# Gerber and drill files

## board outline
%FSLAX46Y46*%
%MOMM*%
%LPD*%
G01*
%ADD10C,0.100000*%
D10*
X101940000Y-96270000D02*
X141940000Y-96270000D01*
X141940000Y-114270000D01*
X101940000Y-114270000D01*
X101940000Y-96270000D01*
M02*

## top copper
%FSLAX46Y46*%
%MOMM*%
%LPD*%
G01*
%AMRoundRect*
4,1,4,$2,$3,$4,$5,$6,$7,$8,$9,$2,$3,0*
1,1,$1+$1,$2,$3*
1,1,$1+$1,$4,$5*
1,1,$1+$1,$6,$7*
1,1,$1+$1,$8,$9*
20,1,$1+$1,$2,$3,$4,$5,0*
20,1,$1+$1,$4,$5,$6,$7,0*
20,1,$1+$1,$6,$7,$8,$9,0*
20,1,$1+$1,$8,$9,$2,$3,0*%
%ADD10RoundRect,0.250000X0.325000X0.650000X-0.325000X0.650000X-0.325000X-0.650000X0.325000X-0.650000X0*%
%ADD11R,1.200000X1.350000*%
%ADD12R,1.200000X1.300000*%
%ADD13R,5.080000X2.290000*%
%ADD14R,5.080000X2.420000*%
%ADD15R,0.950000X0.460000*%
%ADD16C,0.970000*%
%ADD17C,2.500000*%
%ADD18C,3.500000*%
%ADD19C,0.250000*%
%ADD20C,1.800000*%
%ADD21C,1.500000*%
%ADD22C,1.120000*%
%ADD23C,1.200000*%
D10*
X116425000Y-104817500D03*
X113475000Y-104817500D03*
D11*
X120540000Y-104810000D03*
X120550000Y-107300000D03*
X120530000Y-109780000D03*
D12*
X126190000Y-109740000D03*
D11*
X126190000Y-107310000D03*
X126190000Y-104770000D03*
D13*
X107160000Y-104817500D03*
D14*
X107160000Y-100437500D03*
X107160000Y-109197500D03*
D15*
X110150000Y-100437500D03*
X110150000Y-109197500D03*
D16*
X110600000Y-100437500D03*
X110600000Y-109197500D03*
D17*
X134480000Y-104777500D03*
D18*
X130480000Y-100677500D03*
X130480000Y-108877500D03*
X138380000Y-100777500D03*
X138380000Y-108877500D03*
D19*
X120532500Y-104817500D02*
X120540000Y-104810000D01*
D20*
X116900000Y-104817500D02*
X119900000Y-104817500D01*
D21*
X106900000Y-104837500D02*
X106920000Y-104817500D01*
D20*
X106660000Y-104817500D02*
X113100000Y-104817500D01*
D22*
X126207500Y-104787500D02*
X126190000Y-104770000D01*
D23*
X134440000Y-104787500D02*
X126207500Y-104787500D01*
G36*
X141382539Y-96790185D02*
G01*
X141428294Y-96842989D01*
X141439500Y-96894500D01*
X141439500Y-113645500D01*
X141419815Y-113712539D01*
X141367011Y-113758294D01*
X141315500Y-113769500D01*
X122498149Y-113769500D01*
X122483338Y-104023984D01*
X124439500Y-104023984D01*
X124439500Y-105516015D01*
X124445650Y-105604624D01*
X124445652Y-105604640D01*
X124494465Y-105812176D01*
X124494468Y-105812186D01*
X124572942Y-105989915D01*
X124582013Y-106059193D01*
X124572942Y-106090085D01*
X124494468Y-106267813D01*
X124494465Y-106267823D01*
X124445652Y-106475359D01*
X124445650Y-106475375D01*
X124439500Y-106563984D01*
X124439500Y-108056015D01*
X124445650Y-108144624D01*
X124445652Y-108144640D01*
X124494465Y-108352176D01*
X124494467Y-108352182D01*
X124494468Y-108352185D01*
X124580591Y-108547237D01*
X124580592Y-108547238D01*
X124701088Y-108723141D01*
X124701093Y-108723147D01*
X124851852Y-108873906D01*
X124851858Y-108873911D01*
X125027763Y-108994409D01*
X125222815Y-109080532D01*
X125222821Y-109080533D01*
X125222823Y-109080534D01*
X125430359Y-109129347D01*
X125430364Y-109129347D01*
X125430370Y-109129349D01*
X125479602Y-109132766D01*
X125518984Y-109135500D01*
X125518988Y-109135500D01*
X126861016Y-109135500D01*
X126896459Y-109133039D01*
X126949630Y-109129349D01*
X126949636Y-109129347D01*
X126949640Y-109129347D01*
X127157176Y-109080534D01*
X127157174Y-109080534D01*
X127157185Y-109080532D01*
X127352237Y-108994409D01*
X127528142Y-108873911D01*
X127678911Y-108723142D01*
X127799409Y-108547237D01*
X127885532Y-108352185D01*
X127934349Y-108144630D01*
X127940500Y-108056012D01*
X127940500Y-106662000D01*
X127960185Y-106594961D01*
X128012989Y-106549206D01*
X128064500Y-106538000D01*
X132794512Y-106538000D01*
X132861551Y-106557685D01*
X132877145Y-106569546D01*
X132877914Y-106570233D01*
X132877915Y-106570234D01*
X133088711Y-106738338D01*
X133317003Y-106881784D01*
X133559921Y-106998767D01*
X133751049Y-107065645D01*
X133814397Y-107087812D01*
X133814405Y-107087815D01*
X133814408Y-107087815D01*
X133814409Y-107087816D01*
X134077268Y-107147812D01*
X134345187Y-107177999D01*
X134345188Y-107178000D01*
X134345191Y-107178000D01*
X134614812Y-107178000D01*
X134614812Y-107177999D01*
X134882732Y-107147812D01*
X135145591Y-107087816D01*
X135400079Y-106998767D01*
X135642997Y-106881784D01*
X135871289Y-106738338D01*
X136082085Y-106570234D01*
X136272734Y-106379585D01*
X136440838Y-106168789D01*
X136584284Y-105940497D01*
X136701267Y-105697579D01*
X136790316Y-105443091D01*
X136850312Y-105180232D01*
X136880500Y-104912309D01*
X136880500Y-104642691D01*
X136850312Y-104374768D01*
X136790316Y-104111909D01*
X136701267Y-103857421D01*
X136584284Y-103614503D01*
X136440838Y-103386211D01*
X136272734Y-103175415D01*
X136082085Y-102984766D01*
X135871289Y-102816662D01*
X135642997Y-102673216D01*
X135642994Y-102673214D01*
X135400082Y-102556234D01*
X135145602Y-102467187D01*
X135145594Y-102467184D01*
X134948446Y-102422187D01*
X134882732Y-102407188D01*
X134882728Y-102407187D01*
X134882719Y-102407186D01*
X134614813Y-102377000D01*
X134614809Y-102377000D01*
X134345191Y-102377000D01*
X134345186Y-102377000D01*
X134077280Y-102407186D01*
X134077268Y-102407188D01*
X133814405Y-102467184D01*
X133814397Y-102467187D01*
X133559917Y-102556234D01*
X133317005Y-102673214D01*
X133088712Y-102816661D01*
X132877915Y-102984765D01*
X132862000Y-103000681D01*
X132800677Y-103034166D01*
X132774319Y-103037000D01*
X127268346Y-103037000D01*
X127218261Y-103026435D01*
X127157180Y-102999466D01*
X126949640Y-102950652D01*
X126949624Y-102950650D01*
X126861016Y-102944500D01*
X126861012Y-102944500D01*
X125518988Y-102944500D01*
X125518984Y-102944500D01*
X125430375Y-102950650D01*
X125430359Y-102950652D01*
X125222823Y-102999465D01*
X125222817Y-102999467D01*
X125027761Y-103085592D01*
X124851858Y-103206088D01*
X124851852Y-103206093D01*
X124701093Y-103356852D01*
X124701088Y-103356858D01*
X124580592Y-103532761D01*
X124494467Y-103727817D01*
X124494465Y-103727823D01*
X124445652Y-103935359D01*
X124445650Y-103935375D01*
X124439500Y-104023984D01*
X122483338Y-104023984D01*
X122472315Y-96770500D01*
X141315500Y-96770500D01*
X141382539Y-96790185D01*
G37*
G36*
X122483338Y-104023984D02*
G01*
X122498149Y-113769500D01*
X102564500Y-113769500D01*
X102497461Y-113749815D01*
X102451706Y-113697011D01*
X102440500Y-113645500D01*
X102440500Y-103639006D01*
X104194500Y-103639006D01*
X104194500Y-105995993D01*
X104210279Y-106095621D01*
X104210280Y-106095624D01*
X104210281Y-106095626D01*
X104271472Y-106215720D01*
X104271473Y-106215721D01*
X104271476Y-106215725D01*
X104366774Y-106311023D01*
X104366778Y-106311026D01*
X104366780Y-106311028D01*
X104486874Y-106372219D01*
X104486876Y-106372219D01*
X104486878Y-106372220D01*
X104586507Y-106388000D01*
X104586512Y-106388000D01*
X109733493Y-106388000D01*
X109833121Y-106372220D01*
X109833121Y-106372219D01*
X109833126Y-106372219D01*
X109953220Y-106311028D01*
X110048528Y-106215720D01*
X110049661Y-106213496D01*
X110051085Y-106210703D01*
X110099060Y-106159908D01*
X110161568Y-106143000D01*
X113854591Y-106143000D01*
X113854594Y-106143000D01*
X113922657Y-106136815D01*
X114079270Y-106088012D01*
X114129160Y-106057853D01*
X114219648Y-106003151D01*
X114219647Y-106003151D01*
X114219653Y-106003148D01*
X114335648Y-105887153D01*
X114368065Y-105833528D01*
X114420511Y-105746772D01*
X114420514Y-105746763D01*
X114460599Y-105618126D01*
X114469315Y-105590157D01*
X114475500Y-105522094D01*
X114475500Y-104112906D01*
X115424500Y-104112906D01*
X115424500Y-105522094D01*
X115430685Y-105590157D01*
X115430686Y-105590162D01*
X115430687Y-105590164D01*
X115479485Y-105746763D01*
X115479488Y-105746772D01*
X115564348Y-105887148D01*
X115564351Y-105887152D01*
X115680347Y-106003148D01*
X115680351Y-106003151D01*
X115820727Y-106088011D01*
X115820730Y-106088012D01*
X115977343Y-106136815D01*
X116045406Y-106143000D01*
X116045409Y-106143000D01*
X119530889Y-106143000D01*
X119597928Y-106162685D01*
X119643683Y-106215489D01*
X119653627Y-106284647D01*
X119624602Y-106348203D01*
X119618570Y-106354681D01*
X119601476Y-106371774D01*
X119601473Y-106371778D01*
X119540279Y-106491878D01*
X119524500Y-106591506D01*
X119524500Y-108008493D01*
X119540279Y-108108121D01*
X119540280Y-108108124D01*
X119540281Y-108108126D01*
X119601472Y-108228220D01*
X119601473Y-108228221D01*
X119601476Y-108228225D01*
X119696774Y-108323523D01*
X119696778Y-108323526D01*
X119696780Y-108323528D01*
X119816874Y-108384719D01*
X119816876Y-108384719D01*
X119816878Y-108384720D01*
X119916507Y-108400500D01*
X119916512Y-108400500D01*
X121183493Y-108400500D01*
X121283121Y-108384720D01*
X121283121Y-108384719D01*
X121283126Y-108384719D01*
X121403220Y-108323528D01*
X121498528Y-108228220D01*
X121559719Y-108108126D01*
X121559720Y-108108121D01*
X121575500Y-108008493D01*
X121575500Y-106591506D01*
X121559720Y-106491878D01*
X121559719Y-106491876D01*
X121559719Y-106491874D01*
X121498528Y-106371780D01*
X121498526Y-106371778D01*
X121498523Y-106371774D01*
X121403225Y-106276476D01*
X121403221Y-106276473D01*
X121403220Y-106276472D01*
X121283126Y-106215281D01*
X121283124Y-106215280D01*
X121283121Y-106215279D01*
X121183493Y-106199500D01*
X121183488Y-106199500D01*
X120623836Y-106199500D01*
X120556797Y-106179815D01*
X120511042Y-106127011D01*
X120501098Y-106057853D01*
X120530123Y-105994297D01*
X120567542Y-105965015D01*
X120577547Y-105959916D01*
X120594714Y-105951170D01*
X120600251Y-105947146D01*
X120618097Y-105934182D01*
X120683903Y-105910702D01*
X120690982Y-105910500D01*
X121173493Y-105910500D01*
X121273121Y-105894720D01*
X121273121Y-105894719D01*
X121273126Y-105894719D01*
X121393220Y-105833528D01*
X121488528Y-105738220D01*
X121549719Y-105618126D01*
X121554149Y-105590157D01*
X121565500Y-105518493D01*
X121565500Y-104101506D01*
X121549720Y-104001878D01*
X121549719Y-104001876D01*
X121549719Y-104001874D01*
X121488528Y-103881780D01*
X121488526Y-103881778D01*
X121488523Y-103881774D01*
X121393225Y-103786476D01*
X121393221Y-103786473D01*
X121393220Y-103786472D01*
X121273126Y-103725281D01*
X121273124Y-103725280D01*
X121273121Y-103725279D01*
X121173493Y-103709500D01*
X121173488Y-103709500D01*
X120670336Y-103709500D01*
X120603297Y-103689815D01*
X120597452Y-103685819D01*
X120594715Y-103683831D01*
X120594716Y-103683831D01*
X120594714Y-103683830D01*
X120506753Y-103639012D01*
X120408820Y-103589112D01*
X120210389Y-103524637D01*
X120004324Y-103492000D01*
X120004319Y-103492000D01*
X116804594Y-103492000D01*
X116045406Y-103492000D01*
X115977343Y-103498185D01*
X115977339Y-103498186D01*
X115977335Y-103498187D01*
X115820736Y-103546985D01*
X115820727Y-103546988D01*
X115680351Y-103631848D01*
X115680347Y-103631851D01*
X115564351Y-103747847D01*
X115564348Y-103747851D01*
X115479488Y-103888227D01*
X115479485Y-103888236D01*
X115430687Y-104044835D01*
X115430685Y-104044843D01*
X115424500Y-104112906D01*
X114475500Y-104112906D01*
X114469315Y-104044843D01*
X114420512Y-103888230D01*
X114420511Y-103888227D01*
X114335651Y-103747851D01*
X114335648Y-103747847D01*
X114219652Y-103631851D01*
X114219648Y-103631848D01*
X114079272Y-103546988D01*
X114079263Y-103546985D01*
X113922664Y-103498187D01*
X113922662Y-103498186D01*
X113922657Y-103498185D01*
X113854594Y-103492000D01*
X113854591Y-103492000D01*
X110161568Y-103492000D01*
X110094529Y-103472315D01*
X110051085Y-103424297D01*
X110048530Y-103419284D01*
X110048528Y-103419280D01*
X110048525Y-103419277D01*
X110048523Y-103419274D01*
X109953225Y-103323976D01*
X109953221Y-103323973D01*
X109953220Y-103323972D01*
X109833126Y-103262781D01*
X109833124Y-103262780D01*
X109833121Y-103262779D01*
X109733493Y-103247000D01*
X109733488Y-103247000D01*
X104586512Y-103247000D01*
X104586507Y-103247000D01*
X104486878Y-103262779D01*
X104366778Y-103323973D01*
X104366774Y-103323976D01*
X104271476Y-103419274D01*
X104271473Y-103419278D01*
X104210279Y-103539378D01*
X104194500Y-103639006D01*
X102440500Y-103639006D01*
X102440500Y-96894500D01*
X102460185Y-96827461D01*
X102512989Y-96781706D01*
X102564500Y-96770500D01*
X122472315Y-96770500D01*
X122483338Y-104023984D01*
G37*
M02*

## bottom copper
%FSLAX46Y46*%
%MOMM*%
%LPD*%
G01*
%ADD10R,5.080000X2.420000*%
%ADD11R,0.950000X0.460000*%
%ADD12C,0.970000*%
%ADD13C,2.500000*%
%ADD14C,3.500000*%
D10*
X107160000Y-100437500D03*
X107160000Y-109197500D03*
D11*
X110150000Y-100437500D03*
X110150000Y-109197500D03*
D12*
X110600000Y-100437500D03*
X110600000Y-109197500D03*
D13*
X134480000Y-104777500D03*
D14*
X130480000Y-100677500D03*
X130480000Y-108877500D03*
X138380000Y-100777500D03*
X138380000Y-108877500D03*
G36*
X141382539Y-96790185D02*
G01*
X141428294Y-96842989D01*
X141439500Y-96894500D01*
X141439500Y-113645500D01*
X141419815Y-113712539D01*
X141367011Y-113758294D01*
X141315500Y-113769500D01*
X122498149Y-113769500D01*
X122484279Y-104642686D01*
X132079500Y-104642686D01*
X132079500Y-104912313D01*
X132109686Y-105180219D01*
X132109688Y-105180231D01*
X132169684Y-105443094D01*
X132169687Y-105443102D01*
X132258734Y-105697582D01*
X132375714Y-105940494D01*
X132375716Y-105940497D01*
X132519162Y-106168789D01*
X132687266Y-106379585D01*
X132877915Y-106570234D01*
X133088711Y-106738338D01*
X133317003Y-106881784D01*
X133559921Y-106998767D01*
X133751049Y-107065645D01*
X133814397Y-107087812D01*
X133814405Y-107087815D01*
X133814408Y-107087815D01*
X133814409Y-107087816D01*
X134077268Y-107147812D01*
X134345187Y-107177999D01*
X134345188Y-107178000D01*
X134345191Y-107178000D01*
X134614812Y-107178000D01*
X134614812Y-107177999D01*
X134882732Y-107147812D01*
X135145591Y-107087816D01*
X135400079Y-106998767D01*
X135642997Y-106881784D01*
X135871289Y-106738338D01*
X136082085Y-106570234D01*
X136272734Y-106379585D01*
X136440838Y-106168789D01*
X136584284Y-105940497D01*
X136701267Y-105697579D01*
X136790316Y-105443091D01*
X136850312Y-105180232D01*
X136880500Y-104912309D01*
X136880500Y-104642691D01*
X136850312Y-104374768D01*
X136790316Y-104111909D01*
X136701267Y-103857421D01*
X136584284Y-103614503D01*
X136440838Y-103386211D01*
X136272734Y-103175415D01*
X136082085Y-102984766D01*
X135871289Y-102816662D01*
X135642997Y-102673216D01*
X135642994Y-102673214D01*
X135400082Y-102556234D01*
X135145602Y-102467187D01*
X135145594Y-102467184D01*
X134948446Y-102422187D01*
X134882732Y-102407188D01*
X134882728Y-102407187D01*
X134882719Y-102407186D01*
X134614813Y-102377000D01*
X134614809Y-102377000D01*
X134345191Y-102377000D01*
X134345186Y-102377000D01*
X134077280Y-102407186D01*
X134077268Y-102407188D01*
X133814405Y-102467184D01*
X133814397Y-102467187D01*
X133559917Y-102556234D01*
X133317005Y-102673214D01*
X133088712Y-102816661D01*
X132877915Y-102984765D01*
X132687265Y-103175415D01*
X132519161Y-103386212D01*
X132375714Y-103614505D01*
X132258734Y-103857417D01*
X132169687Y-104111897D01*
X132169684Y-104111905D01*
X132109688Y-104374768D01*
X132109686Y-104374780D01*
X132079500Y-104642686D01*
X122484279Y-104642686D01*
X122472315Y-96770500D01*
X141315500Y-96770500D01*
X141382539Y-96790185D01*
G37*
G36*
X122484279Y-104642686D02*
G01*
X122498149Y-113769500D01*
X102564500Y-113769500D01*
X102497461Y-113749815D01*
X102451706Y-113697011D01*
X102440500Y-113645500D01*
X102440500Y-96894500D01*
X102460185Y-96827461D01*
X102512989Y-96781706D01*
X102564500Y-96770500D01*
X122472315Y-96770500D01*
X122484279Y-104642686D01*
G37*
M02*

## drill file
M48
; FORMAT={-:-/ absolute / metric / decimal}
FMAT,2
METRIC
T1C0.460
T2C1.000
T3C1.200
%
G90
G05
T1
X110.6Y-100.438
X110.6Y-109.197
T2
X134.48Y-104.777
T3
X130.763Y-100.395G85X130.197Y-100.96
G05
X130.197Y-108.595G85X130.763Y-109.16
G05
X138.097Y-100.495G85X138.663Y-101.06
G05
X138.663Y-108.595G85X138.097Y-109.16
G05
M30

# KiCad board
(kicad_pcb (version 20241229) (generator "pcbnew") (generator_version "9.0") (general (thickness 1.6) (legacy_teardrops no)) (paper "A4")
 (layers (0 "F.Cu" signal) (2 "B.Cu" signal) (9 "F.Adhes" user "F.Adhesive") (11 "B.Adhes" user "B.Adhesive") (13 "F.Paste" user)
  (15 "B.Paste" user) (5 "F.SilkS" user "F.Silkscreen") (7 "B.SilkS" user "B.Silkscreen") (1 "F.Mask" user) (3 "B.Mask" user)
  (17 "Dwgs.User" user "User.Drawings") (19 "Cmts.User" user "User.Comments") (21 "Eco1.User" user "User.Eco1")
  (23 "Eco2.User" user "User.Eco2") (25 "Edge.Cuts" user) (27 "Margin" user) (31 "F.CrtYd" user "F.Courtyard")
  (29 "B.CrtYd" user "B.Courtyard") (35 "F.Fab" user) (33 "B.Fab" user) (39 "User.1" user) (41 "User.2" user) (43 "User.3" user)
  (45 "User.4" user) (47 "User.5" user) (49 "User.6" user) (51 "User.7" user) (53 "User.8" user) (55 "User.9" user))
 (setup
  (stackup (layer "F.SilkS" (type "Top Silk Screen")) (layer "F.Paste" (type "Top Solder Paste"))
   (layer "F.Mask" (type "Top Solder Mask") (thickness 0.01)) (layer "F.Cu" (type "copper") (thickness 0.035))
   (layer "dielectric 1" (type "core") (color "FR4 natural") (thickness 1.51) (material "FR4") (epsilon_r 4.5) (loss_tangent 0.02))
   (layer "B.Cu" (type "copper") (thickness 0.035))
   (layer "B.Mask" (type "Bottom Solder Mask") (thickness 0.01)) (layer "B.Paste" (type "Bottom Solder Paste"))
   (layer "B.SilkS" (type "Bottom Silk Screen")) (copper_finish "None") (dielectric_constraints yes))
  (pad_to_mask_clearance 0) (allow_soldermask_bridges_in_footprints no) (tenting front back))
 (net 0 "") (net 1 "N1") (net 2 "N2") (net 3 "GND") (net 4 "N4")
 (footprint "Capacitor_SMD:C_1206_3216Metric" (layer "F.Cu") (at 114.95 104.8175 180)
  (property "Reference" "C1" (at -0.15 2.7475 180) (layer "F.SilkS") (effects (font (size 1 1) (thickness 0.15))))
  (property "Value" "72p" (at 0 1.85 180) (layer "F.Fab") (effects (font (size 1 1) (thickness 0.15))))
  (pad "1" smd roundrect (at -1.475 0 180) (size 1.15 1.8) (layers "F.Cu" "F.Mask" "F.Paste") (roundrect_rratio 0.217391) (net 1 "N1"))
  (pad "2" smd roundrect (at 1.475 0 180) (size 1.15 1.8) (layers "F.Cu" "F.Mask" "F.Paste") (roundrect_rratio 0.217391) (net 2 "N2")))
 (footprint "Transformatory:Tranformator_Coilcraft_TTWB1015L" (layer "F.Cu") (at 120.16 104.23)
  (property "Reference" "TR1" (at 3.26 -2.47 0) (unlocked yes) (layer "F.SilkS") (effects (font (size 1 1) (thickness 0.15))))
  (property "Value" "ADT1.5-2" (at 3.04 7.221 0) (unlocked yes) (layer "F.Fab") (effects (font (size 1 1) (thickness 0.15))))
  (pad "1" smd rect (at 0.38 0.58) (size 1.2 1.35) (layers "F.Cu" "F.Mask" "F.Paste") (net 1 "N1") (thermal_bridge_angle 45))
  (pad "2" smd rect (at 0.39 3.07) (size 1.2 1.35) (layers "F.Cu" "F.Mask" "F.Paste") (thermal_bridge_angle 45))
  (pad "3" smd rect (at 0.37 5.55) (size 1.2 1.35) (layers "F.Cu" "F.Mask" "F.Paste") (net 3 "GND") (thermal_bridge_angle 45))
  (pad "4" smd rect (at 6.03 5.51) (size 1.2 1.3) (layers "F.Cu" "F.Mask" "F.Paste") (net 3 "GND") (thermal_bridge_angle 45))
  (pad "5" smd rect (at 6.03 3.08) (size 1.2 1.35) (layers "F.Cu" "F.Mask" "F.Paste") (thermal_bridge_angle 45))
  (pad "6" smd rect (at 6.03 0.54) (size 1.2 1.35) (layers "F.Cu" "F.Mask" "F.Paste") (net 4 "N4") (thermal_bridge_angle 45)))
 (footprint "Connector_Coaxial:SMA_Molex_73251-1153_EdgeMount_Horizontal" (layer "F.Cu") (at 108.88 104.8175)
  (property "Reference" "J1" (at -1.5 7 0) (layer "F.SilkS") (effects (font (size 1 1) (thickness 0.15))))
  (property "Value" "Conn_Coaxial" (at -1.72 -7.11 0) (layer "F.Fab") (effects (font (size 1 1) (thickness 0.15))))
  (pad "1" smd rect (at -1.72 0) (size 5.08 2.29) (layers "F.Cu" "F.Mask" "F.Paste") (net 2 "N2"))
  (pad "2" smd rect (at -1.72 -4.38) (size 5.08 2.42) (layers "F.Cu" "F.Mask" "F.Paste") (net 3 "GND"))
  (pad "2" smd rect (at -1.72 -4.38) (size 5.08 2.42) (layers "B.Cu" "B.Mask" "B.Paste") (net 3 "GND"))
  (pad "2" smd rect (at -1.72 4.38) (size 5.08 2.42) (layers "F.Cu" "F.Mask" "F.Paste") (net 3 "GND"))
  (pad "2" smd rect (at -1.72 4.38) (size 5.08 2.42) (layers "B.Cu" "B.Mask" "B.Paste") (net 3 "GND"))
  (pad "2" smd rect (at 1.27 -4.38) (size 0.95 0.46) (layers "F.Cu") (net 3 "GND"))
  (pad "2" smd rect (at 1.27 -4.38) (size 0.95 0.46) (layers "B.Cu") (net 3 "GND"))
  (pad "2" smd rect (at 1.27 4.38) (size 0.95 0.46) (layers "F.Cu") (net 3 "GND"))
  (pad "2" smd rect (at 1.27 4.38) (size 0.95 0.46) (layers "B.Cu") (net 3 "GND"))
  (pad "2" thru_hole circle (at 1.72 -4.38) (size 0.97 0.97) (drill 0.46) (layers "*.Cu") (remove_unused_layers no) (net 3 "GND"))
  (pad "2" thru_hole circle (at 1.72 4.38) (size 0.97 0.97) (drill 0.46) (layers "*.Cu") (remove_unused_layers no) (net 3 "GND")))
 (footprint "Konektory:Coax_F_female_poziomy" (layer "F.Cu") (at 134.48 104.7775)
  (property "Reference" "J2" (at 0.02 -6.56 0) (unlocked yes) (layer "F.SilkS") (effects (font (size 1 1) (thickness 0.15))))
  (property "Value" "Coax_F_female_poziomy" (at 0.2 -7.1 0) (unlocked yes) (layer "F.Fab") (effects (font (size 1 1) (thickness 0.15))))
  (pad "1" thru_hole circle (at 0 0) (size 2.5 2.5) (drill 1) (layers "*.Cu" "*.Mask") (remove_unused_layers no) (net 4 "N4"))
  (pad "2" thru_hole circle (at -4 -4.1 315) (size 3.5 3.5) (drill oval 1.2 2) (layers "*.Cu" "*.Mask") (remove_unused_layers no)
   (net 3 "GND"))
  (pad "2" thru_hole circle (at -4 4.1 45) (size 3.5 3.5) (drill oval 1.2 2) (layers "*.Cu" "*.Mask") (remove_unused_layers no)
   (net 3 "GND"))
  (pad "2" thru_hole circle (at 3.9 -4 45) (size 3.5 3.5) (drill oval 1.2 2) (layers "*.Cu" "*.Mask") (remove_unused_layers no)
   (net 3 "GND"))
  (pad "2" thru_hole circle (at 3.9 4.1 315) (size 3.5 3.5) (drill oval 1.2 2) (layers "*.Cu" "*.Mask") (remove_unused_layers no)
   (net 3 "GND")))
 (gr_rect (start 101.94 96.27) (end 141.94 114.27) (stroke (width 0.1) (type default)) (fill no) (layer "Edge.Cuts"))
 (segment (start 120.5325 104.8175) (end 120.54 104.81) (width 0.25) (layer "F.Cu") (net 1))
 (segment (start 116.9 104.8175) (end 119.9 104.8175) (width 1.8) (layer "F.Cu") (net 1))
 (segment (start 106.9 104.8375) (end 106.92 104.8175) (width 1.5) (layer "F.Cu") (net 2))
 (segment (start 106.66 104.8175) (end 113.1 104.8175) (width 1.8) (layer "F.Cu") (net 2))
 (segment (start 126.2075 104.7875) (end 126.19 104.77) (width 1.12) (layer "F.Cu") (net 4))
 (segment (start 134.44 104.7875) (end 126.2075 104.7875) (width 1.2) (layer "F.Cu") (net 4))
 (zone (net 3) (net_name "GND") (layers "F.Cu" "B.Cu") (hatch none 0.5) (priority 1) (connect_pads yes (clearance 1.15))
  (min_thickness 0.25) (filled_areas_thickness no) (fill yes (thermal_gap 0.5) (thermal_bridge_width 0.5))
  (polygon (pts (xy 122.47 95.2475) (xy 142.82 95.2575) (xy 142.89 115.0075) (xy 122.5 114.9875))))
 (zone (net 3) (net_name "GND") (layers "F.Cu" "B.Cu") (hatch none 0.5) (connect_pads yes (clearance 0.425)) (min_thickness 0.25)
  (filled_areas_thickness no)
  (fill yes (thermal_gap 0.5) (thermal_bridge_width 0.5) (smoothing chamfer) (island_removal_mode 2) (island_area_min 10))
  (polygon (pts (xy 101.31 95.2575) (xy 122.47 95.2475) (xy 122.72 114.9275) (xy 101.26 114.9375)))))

